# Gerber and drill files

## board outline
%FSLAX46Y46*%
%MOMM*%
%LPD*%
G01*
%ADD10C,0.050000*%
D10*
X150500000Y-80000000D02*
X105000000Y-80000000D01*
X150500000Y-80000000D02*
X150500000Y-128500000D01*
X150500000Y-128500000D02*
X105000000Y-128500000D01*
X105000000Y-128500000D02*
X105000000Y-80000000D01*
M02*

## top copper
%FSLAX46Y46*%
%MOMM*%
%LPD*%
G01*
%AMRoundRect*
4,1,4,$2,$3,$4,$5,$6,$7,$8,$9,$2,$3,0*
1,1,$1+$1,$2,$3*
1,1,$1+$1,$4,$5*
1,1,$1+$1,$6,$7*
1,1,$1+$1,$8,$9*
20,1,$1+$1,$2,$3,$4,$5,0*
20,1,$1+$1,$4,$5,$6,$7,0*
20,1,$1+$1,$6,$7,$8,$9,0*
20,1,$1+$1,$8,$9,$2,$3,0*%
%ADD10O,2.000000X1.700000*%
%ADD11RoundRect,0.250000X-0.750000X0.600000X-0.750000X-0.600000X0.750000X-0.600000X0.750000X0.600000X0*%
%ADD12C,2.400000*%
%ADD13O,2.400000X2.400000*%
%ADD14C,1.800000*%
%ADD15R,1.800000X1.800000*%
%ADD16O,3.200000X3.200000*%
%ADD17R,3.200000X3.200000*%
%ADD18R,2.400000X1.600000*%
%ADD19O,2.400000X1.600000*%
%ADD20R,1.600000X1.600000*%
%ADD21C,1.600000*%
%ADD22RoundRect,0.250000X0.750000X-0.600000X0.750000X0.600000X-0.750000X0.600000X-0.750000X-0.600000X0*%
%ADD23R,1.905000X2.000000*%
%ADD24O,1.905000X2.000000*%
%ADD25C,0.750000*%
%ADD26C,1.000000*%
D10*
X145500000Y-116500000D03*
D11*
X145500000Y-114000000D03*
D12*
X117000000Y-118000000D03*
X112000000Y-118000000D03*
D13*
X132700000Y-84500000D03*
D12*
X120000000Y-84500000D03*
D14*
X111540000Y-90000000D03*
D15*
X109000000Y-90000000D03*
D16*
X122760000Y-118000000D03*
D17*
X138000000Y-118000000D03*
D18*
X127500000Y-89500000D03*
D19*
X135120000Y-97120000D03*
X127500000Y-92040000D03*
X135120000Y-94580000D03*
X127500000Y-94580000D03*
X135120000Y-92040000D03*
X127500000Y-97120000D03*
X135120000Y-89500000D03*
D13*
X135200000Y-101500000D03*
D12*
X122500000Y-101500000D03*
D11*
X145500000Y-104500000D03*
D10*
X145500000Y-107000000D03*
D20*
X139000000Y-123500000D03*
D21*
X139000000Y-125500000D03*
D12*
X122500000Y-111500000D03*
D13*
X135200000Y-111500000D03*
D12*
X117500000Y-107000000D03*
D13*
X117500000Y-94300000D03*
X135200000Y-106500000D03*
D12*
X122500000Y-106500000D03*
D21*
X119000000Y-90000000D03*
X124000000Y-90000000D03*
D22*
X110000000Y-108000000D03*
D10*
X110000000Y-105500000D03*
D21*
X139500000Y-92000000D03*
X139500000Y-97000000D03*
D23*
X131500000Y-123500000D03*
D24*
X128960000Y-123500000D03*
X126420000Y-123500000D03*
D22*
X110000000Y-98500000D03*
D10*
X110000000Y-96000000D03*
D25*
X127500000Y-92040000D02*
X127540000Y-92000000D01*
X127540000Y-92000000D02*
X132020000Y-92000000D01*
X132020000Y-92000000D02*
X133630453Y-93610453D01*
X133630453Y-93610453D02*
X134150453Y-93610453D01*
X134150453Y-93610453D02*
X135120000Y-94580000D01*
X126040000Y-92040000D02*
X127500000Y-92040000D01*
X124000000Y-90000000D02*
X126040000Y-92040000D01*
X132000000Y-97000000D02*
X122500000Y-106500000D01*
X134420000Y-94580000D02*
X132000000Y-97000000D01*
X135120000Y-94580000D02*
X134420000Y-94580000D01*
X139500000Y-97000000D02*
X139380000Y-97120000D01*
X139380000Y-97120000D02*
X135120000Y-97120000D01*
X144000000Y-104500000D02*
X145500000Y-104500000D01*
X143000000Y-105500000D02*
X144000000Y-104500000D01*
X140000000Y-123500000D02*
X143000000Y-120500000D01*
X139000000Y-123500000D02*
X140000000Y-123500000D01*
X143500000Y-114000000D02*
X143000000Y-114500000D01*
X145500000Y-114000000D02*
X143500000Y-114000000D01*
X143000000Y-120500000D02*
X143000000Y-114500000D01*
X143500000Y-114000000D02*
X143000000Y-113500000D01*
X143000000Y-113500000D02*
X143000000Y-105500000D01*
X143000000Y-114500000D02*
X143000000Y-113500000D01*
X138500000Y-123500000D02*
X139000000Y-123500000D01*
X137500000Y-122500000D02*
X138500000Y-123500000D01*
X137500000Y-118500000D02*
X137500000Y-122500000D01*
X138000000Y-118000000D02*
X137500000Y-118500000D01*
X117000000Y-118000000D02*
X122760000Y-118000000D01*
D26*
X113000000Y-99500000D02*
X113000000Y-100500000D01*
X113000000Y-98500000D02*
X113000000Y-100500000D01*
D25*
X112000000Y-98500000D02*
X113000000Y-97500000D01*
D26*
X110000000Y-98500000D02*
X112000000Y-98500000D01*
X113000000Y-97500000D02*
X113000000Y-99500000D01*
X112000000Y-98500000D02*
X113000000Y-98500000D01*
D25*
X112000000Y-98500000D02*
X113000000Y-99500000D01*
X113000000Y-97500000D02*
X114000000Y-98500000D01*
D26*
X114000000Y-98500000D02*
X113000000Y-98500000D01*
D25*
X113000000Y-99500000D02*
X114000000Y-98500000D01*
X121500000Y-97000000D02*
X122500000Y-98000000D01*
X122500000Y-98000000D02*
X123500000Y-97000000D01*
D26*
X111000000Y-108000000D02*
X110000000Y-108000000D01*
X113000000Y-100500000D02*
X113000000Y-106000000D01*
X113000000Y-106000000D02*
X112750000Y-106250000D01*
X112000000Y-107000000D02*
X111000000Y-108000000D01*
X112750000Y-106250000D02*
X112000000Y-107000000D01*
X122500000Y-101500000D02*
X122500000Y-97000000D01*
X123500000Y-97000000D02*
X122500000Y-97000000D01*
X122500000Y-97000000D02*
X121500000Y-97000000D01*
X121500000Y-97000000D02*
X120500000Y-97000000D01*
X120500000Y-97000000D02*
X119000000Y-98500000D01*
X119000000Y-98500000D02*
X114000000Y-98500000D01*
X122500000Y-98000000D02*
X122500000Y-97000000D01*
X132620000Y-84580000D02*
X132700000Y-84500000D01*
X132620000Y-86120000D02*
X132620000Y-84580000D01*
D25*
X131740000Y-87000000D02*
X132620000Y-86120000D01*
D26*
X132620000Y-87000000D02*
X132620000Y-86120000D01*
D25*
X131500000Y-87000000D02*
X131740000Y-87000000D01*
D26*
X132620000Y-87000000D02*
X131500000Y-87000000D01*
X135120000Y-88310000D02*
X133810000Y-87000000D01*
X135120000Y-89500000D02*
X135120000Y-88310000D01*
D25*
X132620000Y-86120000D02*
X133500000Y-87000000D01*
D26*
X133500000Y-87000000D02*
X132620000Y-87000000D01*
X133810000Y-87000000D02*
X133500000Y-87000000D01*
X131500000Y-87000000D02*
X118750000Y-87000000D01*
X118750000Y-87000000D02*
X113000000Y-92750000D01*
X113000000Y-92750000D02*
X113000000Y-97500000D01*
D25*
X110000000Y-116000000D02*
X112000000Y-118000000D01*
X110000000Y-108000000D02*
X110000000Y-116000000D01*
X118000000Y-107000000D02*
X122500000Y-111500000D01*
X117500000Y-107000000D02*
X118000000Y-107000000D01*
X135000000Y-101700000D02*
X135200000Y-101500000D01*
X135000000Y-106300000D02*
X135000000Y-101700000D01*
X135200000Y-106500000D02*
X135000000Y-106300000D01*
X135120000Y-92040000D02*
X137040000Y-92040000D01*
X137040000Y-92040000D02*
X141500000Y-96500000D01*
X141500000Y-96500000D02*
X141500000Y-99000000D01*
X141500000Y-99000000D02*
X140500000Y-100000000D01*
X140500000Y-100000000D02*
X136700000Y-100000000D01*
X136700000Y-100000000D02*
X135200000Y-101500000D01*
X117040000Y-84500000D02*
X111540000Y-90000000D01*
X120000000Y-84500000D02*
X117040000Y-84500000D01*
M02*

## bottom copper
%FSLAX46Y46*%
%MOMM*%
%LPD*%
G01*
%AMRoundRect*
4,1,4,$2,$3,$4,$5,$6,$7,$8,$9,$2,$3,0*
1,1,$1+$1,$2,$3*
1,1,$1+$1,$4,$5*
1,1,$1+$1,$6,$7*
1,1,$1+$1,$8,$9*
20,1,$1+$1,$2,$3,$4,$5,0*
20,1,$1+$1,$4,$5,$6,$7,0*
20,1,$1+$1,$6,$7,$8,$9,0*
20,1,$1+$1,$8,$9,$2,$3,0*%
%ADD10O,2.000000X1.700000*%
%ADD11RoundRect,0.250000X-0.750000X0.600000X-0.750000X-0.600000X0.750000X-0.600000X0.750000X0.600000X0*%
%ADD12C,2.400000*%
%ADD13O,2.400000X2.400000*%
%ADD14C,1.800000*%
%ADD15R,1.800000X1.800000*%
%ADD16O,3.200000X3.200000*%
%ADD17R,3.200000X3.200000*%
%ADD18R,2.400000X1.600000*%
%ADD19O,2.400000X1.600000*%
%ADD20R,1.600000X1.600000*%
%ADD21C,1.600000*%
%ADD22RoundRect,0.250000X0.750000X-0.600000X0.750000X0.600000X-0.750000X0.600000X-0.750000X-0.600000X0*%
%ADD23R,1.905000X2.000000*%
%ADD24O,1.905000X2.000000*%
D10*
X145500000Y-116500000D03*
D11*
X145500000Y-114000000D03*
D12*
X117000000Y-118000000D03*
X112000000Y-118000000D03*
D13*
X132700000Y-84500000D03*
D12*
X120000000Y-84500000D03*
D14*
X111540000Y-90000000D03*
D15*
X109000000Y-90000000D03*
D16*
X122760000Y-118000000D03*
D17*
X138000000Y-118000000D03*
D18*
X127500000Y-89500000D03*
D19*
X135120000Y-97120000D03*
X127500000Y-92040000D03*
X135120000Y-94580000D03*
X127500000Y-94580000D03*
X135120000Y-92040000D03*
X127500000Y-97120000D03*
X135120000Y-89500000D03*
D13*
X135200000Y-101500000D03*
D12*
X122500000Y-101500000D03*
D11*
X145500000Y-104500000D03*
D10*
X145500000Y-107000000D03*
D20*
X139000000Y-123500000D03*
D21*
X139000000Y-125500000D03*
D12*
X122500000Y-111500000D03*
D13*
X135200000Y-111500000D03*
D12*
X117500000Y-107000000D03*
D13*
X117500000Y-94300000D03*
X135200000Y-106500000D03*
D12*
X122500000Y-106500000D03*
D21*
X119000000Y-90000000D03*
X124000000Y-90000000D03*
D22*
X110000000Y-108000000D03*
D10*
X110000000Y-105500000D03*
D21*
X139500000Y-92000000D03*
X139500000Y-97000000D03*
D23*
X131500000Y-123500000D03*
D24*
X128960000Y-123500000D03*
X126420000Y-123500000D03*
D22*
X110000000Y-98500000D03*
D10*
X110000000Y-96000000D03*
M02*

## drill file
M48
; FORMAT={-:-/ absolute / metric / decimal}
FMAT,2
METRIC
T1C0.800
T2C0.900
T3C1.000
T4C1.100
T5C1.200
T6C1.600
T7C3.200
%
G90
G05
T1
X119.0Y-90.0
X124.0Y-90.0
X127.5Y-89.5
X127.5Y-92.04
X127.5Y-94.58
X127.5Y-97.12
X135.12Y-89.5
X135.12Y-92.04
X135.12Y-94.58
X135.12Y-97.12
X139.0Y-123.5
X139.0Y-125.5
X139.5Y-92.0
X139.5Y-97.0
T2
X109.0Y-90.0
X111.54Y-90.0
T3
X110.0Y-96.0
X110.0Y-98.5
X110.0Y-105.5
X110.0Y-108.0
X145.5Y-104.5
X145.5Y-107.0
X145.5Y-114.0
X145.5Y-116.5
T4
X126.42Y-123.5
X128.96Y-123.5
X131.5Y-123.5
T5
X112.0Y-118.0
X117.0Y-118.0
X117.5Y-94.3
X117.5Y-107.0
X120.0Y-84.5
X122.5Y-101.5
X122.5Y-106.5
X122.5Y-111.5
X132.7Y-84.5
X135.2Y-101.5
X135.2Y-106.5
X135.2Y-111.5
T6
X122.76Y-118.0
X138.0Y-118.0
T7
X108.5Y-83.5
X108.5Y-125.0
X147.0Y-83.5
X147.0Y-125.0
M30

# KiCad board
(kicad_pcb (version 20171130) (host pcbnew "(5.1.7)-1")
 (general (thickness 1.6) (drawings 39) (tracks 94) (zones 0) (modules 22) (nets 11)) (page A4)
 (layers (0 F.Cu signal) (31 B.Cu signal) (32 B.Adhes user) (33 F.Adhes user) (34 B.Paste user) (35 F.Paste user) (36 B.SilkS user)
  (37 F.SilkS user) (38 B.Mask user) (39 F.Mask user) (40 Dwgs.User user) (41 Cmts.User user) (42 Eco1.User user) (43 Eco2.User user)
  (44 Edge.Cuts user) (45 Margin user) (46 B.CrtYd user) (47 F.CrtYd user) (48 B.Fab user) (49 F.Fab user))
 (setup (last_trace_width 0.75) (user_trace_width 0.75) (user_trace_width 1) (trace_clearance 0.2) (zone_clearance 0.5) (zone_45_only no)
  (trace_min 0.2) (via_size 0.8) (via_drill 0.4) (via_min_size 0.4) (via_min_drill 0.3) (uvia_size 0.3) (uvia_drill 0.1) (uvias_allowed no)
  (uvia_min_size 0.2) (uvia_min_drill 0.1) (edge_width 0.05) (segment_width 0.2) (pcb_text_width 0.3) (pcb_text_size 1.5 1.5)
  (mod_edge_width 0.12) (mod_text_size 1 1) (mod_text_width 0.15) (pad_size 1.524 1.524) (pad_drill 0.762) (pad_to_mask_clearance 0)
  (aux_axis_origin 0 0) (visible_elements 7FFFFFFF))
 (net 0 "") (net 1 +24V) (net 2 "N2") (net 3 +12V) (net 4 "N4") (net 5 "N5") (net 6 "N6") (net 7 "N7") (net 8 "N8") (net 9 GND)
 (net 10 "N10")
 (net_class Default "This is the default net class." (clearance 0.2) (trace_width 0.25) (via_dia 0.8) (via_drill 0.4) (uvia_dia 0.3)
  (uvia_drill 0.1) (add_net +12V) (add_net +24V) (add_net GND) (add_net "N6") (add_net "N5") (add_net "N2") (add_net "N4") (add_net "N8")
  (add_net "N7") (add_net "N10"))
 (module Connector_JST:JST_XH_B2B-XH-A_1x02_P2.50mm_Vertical (layer F.Cu) (at 145.5 114 270)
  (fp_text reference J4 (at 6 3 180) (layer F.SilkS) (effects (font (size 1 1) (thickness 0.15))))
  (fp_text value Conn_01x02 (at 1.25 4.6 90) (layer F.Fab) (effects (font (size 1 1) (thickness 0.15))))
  (pad 2 thru_hole oval (at 2.5 0 270) (size 1.7 2) (drill 1) (layers *.Cu *.Mask))
  (pad 1 thru_hole roundrect (at 0 0 270) (size 1.7 2) (drill 1) (layers *.Cu *.Mask) (roundrect_rratio 0.147059) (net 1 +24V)))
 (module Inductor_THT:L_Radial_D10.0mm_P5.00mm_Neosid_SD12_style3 (layer F.Cu) (at 112 118)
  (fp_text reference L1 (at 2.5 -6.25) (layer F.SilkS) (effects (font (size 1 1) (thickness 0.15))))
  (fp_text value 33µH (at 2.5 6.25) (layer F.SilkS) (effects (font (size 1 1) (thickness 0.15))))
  (pad 2 thru_hole circle (at 5 0) (size 2.4 2.4) (drill 1.2) (layers *.Cu *.Mask) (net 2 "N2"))
  (pad 1 thru_hole circle (at 0 0) (size 2.4 2.4) (drill 1.2) (layers *.Cu *.Mask) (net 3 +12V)))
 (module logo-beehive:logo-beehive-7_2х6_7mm (layer F.Cu) (at 139 85)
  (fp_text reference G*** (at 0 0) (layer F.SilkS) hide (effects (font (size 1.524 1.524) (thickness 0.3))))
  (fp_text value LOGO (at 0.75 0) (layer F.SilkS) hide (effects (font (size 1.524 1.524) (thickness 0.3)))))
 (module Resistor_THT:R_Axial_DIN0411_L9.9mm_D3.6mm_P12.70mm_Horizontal (layer F.Cu) (at 120 84.5)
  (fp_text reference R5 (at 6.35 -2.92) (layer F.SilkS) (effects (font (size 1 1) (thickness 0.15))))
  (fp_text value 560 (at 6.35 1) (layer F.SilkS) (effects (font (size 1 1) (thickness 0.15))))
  (pad 2 thru_hole oval (at 12.7 0) (size 2.4 2.4) (drill 1.2) (layers *.Cu *.Mask) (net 3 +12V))
  (pad 1 thru_hole circle (at 0 0) (size 2.4 2.4) (drill 1.2) (layers *.Cu *.Mask) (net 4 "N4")))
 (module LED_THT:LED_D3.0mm (layer F.Cu) (at 109 90)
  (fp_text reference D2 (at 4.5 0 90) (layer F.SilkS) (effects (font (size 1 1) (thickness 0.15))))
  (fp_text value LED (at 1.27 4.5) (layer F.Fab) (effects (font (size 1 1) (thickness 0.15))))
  (pad 2 thru_hole circle (at 2.54 0) (size 1.8 1.8) (drill 0.9) (layers *.Cu *.Mask) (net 4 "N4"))
  (pad 1 thru_hole rect (at 0 0) (size 1.8 1.8) (drill 0.9) (layers *.Cu *.Mask)))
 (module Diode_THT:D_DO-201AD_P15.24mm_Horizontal (layer F.Cu) (at 138 118 180)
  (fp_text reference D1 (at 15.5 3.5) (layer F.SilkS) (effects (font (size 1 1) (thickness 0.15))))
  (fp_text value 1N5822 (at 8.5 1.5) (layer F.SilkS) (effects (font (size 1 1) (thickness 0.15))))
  (pad 2 thru_hole oval (at 15.24 0 180) (size 3.2 3.2) (drill 1.6) (layers *.Cu *.Mask) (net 2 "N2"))
  (pad 1 thru_hole rect (at 0 0 180) (size 3.2 3.2) (drill 1.6) (layers *.Cu *.Mask) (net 1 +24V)))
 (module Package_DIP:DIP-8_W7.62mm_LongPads (layer F.Cu) (at 127.5 89.5)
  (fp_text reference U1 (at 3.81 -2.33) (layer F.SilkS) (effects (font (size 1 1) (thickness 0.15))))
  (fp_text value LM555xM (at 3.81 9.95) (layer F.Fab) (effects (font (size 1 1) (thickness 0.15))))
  (pad 1 thru_hole rect (at 0 0) (size 2.4 1.6) (drill 0.8) (layers *.Cu *.Mask))
  (pad 5 thru_hole oval (at 7.62 7.62) (size 2.4 1.6) (drill 0.8) (layers *.Cu *.Mask) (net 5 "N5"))
  (pad 2 thru_hole oval (at 0 2.54) (size 2.4 1.6) (drill 0.8) (layers *.Cu *.Mask) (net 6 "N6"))
  (pad 6 thru_hole oval (at 7.62 5.08) (size 2.4 1.6) (drill 0.8) (layers *.Cu *.Mask) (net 6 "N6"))
  (pad 3 thru_hole oval (at 0 5.08) (size 2.4 1.6) (drill 0.8) (layers *.Cu *.Mask))
  (pad 7 thru_hole oval (at 7.62 2.54) (size 2.4 1.6) (drill 0.8) (layers *.Cu *.Mask) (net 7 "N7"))
  (pad 4 thru_hole oval (at 0 7.62) (size 2.4 1.6) (drill 0.8) (layers *.Cu *.Mask))
  (pad 8 thru_hole oval (at 7.62 0) (size 2.4 1.6) (drill 0.8) (layers *.Cu *.Mask) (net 3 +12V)))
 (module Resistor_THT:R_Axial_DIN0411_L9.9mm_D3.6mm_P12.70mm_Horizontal (layer F.Cu) (at 122.5 101.5)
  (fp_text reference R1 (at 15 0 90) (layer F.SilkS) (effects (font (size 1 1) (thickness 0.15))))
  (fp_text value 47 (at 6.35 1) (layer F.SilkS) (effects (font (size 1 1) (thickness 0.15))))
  (pad 2 thru_hole oval (at 12.7 0) (size 2.4 2.4) (drill 1.2) (layers *.Cu *.Mask) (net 7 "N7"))
  (pad 1 thru_hole circle (at 0 0) (size 2.4 2.4) (drill 1.2) (layers *.Cu *.Mask) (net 3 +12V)))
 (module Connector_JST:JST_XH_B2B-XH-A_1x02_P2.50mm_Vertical (layer F.Cu) (at 145.5 104.5 270)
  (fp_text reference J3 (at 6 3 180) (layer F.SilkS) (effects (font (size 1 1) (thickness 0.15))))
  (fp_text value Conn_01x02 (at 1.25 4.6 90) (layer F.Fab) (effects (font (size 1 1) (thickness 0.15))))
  (pad 1 thru_hole roundrect (at 0 0 270) (size 1.7 2) (drill 1) (layers *.Cu *.Mask) (roundrect_rratio 0.1470588235294118) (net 1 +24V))
  (pad 2 thru_hole oval (at 2.5 0 270) (size 1.7 2) (drill 1) (layers *.Cu *.Mask)))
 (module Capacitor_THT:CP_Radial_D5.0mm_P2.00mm (layer F.Cu) (at 139 123.5 270)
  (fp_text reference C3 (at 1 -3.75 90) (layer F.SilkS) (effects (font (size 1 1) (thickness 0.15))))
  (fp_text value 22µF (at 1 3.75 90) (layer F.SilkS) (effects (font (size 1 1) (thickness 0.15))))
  (pad 1 thru_hole rect (at 0 0 270) (size 1.6 1.6) (drill 0.8) (layers *.Cu *.Mask) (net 1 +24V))
  (pad 2 thru_hole circle (at 2 0 270) (size 1.6 1.6) (drill 0.8) (layers *.Cu *.Mask)))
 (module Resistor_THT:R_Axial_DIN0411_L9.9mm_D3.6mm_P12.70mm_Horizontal (layer F.Cu) (at 122.5 111.5)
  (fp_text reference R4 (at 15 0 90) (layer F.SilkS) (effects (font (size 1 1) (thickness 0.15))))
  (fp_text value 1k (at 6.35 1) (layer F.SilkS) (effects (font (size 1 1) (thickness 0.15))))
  (pad 1 thru_hole circle (at 0 0) (size 2.4 2.4) (drill 1.2) (layers *.Cu *.Mask) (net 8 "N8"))
  (pad 2 thru_hole oval (at 12.7 0) (size 2.4 2.4) (drill 1.2) (layers *.Cu *.Mask)))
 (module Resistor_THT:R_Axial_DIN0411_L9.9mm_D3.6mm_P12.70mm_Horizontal (layer F.Cu) (at 117.5 107 90)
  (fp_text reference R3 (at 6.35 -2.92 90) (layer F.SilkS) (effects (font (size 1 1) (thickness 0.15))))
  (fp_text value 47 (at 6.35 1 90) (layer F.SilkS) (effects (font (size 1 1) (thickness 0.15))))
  (pad 1 thru_hole circle (at 0 0 90) (size 2.4 2.4) (drill 1.2) (layers *.Cu *.Mask) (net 8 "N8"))
  (pad 2 thru_hole oval (at 12.7 0 90) (size 2.4 2.4) (drill 1.2) (layers *.Cu *.Mask)))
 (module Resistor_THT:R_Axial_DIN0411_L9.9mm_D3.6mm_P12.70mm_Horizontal (layer F.Cu) (at 122.5 106.5)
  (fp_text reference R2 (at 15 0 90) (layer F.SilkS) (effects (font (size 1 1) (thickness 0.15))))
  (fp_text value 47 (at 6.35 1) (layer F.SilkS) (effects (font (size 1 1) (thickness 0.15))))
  (pad 2 thru_hole oval (at 12.7 0) (size 2.4 2.4) (drill 1.2) (layers *.Cu *.Mask) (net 7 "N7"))
  (pad 1 thru_hole circle (at 0 0) (size 2.4 2.4) (drill 1.2) (layers *.Cu *.Mask) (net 6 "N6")))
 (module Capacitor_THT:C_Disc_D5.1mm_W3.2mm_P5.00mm (layer F.Cu) (at 119 90)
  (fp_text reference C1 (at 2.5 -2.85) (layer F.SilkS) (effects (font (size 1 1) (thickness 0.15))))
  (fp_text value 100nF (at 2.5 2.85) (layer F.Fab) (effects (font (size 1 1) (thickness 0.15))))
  (pad 1 thru_hole circle (at 0 0) (size 1.6 1.6) (drill 0.8) (layers *.Cu *.Mask))
  (pad 2 thru_hole circle (at 5 0) (size 1.6 1.6) (drill 0.8) (layers *.Cu *.Mask) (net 6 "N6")))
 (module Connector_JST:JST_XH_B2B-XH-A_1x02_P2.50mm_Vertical (layer F.Cu) (at 110 108 90)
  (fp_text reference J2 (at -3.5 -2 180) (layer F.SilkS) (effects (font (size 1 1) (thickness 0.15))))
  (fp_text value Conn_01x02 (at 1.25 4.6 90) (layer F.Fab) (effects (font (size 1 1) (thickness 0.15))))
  (pad 1 thru_hole roundrect (at 0 0 90) (size 1.7 2) (drill 1) (layers *.Cu *.Mask) (roundrect_rratio 0.1470588235294118) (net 3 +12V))
  (pad 2 thru_hole oval (at 2.5 0 90) (size 1.7 2) (drill 1) (layers *.Cu *.Mask)))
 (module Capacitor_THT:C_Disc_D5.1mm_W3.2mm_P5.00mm (layer F.Cu) (at 139.5 92 270)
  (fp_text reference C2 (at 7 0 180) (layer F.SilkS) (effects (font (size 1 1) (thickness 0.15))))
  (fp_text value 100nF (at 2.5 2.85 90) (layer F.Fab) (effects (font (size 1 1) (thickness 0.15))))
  (pad 1 thru_hole circle (at 0 0 270) (size 1.6 1.6) (drill 0.8) (layers *.Cu *.Mask))
  (pad 2 thru_hole circle (at 5 0 270) (size 1.6 1.6) (drill 0.8) (layers *.Cu *.Mask) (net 5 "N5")))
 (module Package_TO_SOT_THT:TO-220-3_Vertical (layer F.Cu) (at 131.5 123.5 180)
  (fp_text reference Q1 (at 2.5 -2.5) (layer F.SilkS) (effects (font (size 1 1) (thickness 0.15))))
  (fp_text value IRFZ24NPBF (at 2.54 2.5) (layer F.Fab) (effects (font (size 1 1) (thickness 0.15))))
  (pad 1 thru_hole rect (at 0 0 180) (size 1.905 2) (drill 1.1) (layers *.Cu *.Mask))
  (pad 2 thru_hole oval (at 2.54 0 180) (size 1.905 2) (drill 1.1) (layers *.Cu *.Mask))
  (pad 3 thru_hole oval (at 5.08 0 180) (size 1.905 2) (drill 1.1) (layers *.Cu *.Mask)))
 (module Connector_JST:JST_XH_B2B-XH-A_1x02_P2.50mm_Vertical (layer F.Cu) (at 110 98.5 90)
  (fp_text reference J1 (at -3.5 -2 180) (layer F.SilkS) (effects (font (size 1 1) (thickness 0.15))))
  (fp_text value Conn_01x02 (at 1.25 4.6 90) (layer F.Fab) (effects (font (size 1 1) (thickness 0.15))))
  (pad 1 thru_hole roundrect (at 0 0 90) (size 1.7 2) (drill 1) (layers *.Cu *.Mask) (roundrect_rratio 0.1470588235294118) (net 3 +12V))
  (pad 2 thru_hole oval (at 2.5 0 90) (size 1.7 2) (drill 1) (layers *.Cu *.Mask)))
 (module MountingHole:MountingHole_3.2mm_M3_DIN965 (layer F.Cu) (at 147 83.5)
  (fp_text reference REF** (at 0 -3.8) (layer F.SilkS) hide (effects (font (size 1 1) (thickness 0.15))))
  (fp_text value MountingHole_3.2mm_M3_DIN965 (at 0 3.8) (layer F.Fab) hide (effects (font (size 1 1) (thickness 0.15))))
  (pad 1 np_thru_hole circle (at 0 0) (size 3.2 3.2) (drill 3.2) (layers *.Cu *.Mask)))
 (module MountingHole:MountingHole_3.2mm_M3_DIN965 (layer F.Cu) (at 108.5 125)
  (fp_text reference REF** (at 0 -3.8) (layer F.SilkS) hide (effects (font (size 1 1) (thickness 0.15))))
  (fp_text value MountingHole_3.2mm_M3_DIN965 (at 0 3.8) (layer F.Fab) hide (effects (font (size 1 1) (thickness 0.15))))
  (pad 1 np_thru_hole circle (at 0 0) (size 3.2 3.2) (drill 3.2) (layers *.Cu *.Mask)))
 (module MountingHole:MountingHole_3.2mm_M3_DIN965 (layer F.Cu) (at 147 125)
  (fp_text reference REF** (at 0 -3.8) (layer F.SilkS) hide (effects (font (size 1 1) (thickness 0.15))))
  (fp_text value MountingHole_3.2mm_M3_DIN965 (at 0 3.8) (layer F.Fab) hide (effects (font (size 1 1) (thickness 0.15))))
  (pad 1 np_thru_hole circle (at 0 0) (size 3.2 3.2) (drill 3.2) (layers *.Cu *.Mask)))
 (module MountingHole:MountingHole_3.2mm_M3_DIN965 (layer F.Cu) (at 108.5 83.5)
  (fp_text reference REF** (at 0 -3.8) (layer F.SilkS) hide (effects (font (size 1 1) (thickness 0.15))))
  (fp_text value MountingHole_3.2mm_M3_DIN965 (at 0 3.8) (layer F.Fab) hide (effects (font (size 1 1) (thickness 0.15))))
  (pad 1 np_thru_hole circle (at 0 0) (size 3.2 3.2) (drill 3.2) (layers *.Cu *.Mask)))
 (gr_line (start 150.5 80) (end 105 80) (layer Edge.Cuts) (width 0.05))
 (gr_line (start 150.5 80) (end 150.5 128.5) (layer Edge.Cuts) (width 0.05))
 (gr_line (start 150.5 128.5) (end 105 128.5) (layer Edge.Cuts) (width 0.05))
 (gr_line (start 105 128.5) (end 105 80) (layer Edge.Cuts) (width 0.05))
 (segment (start 127.5 92.04) (end 127.54 92) (width 0.75) (layer F.Cu) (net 6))
 (segment (start 127.54 92) (end 132.02 92) (width 0.75) (layer F.Cu) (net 6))
 (segment (start 132.02 92) (end 133.630453 93.610453) (width 0.75) (layer F.Cu) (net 6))
 (segment (start 133.630453 93.610453) (end 134.150453 93.610453) (width 0.75) (layer F.Cu) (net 6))
 (segment (start 134.150453 93.610453) (end 135.12 94.58) (width 0.75) (layer F.Cu) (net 6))
 (segment (start 126.04 92.04) (end 127.5 92.04) (width 0.75) (layer F.Cu) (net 6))
 (segment (start 124 90) (end 126.04 92.04) (width 0.75) (layer F.Cu) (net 6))
 (segment (start 132 97) (end 122.5 106.5) (width 0.75) (layer F.Cu) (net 6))
 (segment (start 134.42 94.58) (end 132 97) (width 0.75) (layer F.Cu) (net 6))
 (segment (start 135.12 94.58) (end 134.42 94.58) (width 0.75) (layer F.Cu) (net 6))
 (segment (start 139.5 97) (end 139.38 97.12) (width 0.75) (layer F.Cu) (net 5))
 (segment (start 139.38 97.12) (end 135.12 97.12) (width 0.75) (layer F.Cu) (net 5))
 (segment (start 144 104.5) (end 145.5 104.5) (width 0.75) (layer F.Cu) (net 1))
 (segment (start 143 105.5) (end 144 104.5) (width 0.75) (layer F.Cu) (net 1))
 (segment (start 140 123.5) (end 143 120.5) (width 0.75) (layer F.Cu) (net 1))
 (segment (start 139 123.5) (end 140 123.5) (width 0.75) (layer F.Cu) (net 1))
 (segment (start 143.5 114) (end 143 114.5) (width 0.75) (layer F.Cu) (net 1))
 (segment (start 145.5 114) (end 143.5 114) (width 0.75) (layer F.Cu) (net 1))
 (segment (start 143 120.5) (end 143 114.5) (width 0.75) (layer F.Cu) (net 1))
 (segment (start 143.5 114) (end 143 113.5) (width 0.75) (layer F.Cu) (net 1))
 (segment (start 143 113.5) (end 143 105.5) (width 0.75) (layer F.Cu) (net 1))
 (segment (start 143 114.5) (end 143 113.5) (width 0.75) (layer F.Cu) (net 1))
 (segment (start 138.5 123.5) (end 139 123.5) (width 0.75) (layer F.Cu) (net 1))
 (segment (start 137.5 122.5) (end 138.5 123.5) (width 0.75) (layer F.Cu) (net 1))
 (segment (start 137.5 118.5) (end 137.5 122.5) (width 0.75) (layer F.Cu) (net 1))
 (segment (start 138 118) (end 137.5 118.5) (width 0.75) (layer F.Cu) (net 1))
 (segment (start 117 118) (end 122.76 118) (width 0.75) (layer F.Cu) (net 2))
 (segment (start 113 99.5) (end 113 100.5) (width 1) (layer F.Cu) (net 3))
 (segment (start 113 98.5) (end 113 100.5) (width 1) (layer F.Cu) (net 3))
 (segment (start 112 98.5) (end 113 97.5) (width 0.75) (layer F.Cu) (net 3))
 (segment (start 110 98.5) (end 112 98.5) (width 1) (layer F.Cu) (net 3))
 (segment (start 113 97.5) (end 113 99.5) (width 1) (layer F.Cu) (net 3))
 (segment (start 112 98.5) (end 113 98.5) (width 1) (layer F.Cu) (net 3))
 (segment (start 112 98.5) (end 113 99.5) (width 0.75) (layer F.Cu) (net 3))
 (segment (start 113 97.5) (end 114 98.5) (width 0.75) (layer F.Cu) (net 3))
 (segment (start 114 98.5) (end 113 98.5) (width 1) (layer F.Cu) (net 3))
 (segment (start 113 99.5) (end 114 98.5) (width 0.75) (layer F.Cu) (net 3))
 (segment (start 121.5 97) (end 122.5 98) (width 0.75) (layer F.Cu) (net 3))
 (segment (start 122.5 98) (end 123.5 97) (width 0.75) (layer F.Cu) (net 3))
 (segment (start 111 108) (end 110 108) (width 1) (layer F.Cu) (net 3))
 (segment (start 113 100.5) (end 113 106) (width 1) (layer F.Cu) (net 3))
 (segment (start 113 106) (end 112.75 106.25) (width 1) (layer F.Cu) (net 3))
 (segment (start 112 107) (end 111 108) (width 1) (layer F.Cu) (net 3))
 (segment (start 112.75 106.25) (end 112 107) (width 1) (layer F.Cu) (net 3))
 (segment (start 122.5 101.5) (end 122.5 97) (width 1) (layer F.Cu) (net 3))
 (segment (start 123.5 97) (end 122.5 97) (width 1) (layer F.Cu) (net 3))
 (segment (start 122.5 97) (end 121.5 97) (width 1) (layer F.Cu) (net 3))
 (segment (start 121.5 97) (end 120.5 97) (width 1) (layer F.Cu) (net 3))
 (segment (start 120.5 97) (end 119 98.5) (width 1) (layer F.Cu) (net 3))
 (segment (start 119 98.5) (end 114 98.5) (width 1) (layer F.Cu) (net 3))
 (segment (start 122.5 98) (end 122.5 97) (width 1) (layer F.Cu) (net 3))
 (segment (start 132.62 84.58) (end 132.7 84.5) (width 1) (layer F.Cu) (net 3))
 (segment (start 132.62 86.12) (end 132.62 84.58) (width 1) (layer F.Cu) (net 3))
 (segment (start 131.74 87) (end 132.62 86.12) (width 0.75) (layer F.Cu) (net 3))
 (segment (start 132.62 87) (end 132.62 86.12) (width 1) (layer F.Cu) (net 3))
 (segment (start 131.5 87) (end 131.74 87) (width 0.75) (layer F.Cu) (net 3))
 (segment (start 132.62 87) (end 131.5 87) (width 1) (layer F.Cu) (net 3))
 (segment (start 135.12 88.31) (end 133.81 87) (width 1) (layer F.Cu) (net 3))
 (segment (start 135.12 89.5) (end 135.12 88.31) (width 1) (layer F.Cu) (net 3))
 (segment (start 132.62 86.12) (end 133.5 87) (width 0.75) (layer F.Cu) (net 3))
 (segment (start 133.5 87) (end 132.62 87) (width 1) (layer F.Cu) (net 3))
 (segment (start 133.81 87) (end 133.5 87) (width 1) (layer F.Cu) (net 3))
 (segment (start 131.5 87) (end 118.75 87) (width 1) (layer F.Cu) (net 3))
 (segment (start 118.75 87) (end 113 92.75) (width 1) (layer F.Cu) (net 3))
 (segment (start 113 92.75) (end 113 97.5) (width 1) (layer F.Cu) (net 3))
 (segment (start 110 116) (end 112 118) (width 0.75) (layer F.Cu) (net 3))
 (segment (start 110 108) (end 110 116) (width 0.75) (layer F.Cu) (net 3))
 (segment (start 118 107) (end 122.5 111.5) (width 0.75) (layer F.Cu) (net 8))
 (segment (start 117.5 107) (end 118 107) (width 0.75) (layer F.Cu) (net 8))
 (segment (start 135 101.7) (end 135.2 101.5) (width 0.75) (layer F.Cu) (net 7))
 (segment (start 135 106.3) (end 135 101.7) (width 0.75) (layer F.Cu) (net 7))
 (segment (start 135.2 106.5) (end 135 106.3) (width 0.75) (layer F.Cu) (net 7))
 (segment (start 135.12 92.04) (end 137.04 92.04) (width 0.75) (layer F.Cu) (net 7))
 (segment (start 137.04 92.04) (end 141.5 96.5) (width 0.75) (layer F.Cu) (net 7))
 (segment (start 141.5 96.5) (end 141.5 99) (width 0.75) (layer F.Cu) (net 7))
 (segment (start 141.5 99) (end 140.5 100) (width 0.75) (layer F.Cu) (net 7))
 (segment (start 140.5 100) (end 136.7 100) (width 0.75) (layer F.Cu) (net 7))
 (segment (start 136.7 100) (end 135.2 101.5) (width 0.75) (layer F.Cu) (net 7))
 (segment (start 117.04 84.5) (end 111.54 90) (width 0.75) (layer F.Cu) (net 4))
 (segment (start 120 84.5) (end 117.04 84.5) (width 0.75) (layer F.Cu) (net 4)))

